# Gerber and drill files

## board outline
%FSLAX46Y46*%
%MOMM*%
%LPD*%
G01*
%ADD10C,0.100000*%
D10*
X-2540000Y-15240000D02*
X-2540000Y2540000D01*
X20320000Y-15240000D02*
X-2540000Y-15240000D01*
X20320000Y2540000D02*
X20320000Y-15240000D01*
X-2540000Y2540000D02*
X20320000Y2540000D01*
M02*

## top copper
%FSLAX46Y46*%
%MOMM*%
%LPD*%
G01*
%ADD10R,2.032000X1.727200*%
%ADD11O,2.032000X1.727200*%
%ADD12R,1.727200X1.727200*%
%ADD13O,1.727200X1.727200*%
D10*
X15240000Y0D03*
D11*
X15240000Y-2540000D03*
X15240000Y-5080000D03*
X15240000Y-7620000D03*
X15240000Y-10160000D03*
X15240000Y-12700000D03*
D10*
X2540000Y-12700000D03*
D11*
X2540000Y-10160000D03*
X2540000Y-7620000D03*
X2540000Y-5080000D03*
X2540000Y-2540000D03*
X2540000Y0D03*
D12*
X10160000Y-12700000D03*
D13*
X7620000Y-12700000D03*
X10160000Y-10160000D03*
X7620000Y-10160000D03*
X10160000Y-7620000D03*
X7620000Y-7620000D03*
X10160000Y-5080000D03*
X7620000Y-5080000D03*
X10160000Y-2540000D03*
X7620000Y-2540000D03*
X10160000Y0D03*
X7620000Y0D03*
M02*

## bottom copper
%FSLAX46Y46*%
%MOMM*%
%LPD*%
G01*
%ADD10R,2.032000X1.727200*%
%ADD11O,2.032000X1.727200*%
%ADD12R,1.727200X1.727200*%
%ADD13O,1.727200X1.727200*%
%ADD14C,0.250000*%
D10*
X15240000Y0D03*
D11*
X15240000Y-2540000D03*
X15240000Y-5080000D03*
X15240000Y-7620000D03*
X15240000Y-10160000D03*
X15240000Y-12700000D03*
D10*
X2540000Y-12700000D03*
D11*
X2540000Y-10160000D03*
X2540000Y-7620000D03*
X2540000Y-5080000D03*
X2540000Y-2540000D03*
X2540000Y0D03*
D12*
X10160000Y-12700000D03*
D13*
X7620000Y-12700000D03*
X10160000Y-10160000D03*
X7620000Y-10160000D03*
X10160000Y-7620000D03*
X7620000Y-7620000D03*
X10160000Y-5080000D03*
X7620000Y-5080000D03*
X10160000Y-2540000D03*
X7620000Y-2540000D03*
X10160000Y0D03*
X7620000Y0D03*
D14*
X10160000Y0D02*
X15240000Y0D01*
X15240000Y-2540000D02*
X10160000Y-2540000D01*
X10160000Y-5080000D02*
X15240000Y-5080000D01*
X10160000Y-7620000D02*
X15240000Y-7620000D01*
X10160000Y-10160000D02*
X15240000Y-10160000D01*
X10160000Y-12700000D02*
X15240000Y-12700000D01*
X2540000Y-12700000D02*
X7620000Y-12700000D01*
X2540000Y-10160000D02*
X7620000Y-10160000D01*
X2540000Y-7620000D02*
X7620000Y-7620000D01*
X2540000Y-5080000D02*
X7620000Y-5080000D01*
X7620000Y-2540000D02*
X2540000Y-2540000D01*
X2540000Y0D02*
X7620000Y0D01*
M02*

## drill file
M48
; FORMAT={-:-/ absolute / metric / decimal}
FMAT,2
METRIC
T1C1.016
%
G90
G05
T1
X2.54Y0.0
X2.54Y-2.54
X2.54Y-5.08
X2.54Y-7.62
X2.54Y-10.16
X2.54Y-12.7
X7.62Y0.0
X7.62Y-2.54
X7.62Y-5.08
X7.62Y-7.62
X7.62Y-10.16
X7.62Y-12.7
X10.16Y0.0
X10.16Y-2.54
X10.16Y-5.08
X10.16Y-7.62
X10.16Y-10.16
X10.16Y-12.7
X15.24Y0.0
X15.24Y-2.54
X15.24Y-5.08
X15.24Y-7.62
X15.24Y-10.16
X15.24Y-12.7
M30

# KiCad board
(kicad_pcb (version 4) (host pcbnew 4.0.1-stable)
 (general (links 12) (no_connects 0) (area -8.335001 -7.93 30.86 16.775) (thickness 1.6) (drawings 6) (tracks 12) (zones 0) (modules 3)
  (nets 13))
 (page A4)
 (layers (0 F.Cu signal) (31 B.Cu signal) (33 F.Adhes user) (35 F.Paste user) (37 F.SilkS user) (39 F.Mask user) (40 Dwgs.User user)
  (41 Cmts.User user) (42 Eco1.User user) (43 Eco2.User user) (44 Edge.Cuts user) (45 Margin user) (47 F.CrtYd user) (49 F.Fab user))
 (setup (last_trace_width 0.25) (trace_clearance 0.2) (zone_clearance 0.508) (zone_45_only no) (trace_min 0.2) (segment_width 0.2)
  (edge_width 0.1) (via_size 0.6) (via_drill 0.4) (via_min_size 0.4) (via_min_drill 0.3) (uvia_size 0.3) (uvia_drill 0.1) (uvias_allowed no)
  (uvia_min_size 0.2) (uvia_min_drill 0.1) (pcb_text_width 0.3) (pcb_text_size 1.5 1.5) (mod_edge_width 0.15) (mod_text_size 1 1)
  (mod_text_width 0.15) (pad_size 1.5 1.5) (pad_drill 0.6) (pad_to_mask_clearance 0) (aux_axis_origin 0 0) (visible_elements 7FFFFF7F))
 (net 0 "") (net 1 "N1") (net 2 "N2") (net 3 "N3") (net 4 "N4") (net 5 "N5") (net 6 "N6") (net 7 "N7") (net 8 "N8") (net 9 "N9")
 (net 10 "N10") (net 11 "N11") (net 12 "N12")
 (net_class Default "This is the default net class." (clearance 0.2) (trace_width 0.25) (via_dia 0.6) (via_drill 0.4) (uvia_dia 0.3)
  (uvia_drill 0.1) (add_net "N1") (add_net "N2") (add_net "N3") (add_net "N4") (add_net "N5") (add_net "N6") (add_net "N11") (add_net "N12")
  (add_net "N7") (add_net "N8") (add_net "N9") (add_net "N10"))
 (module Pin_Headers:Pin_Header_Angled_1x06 (layer F.Cu) (at 15.24 0)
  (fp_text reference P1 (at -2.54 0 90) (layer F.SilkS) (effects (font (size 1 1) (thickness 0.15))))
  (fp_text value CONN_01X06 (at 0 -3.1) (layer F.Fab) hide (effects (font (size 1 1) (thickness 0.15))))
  (pad 1 thru_hole rect (at 0 0) (size 2.032 1.7272) (drill 1.016) (layers *.Cu *.Mask) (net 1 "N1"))
  (pad 2 thru_hole oval (at 0 2.54) (size 2.032 1.7272) (drill 1.016) (layers *.Cu *.Mask) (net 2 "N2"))
  (pad 3 thru_hole oval (at 0 5.08) (size 2.032 1.7272) (drill 1.016) (layers *.Cu *.Mask) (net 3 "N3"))
  (pad 4 thru_hole oval (at 0 7.62) (size 2.032 1.7272) (drill 1.016) (layers *.Cu *.Mask) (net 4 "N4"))
  (pad 5 thru_hole oval (at 0 10.16) (size 2.032 1.7272) (drill 1.016) (layers *.Cu *.Mask) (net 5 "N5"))
  (pad 6 thru_hole oval (at 0 12.7) (size 2.032 1.7272) (drill 1.016) (layers *.Cu *.Mask) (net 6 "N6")))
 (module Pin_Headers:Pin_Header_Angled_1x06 (layer F.Cu) (at 2.54 12.7 180)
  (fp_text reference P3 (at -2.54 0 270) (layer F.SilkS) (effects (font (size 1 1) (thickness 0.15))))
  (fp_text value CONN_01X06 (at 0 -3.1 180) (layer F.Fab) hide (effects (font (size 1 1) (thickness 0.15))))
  (pad 1 thru_hole rect (at 0 0 180) (size 2.032 1.7272) (drill 1.016) (layers *.Cu *.Mask) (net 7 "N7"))
  (pad 2 thru_hole oval (at 0 2.54 180) (size 2.032 1.7272) (drill 1.016) (layers *.Cu *.Mask) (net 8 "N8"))
  (pad 3 thru_hole oval (at 0 5.08 180) (size 2.032 1.7272) (drill 1.016) (layers *.Cu *.Mask) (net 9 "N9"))
  (pad 4 thru_hole oval (at 0 7.62 180) (size 2.032 1.7272) (drill 1.016) (layers *.Cu *.Mask) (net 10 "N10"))
  (pad 5 thru_hole oval (at 0 10.16 180) (size 2.032 1.7272) (drill 1.016) (layers *.Cu *.Mask) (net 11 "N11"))
  (pad 6 thru_hole oval (at 0 12.7 180) (size 2.032 1.7272) (drill 1.016) (layers *.Cu *.Mask) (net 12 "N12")))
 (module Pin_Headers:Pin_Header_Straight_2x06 (layer F.Cu) (at 10.16 12.7 180)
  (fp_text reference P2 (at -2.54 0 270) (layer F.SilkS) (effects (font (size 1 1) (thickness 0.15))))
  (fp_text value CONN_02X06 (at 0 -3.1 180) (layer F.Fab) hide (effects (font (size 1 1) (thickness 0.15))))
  (pad 1 thru_hole rect (at 0 0 180) (size 1.7272 1.7272) (drill 1.016) (layers *.Cu *.Mask) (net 6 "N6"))
  (pad 2 thru_hole oval (at 2.54 0 180) (size 1.7272 1.7272) (drill 1.016) (layers *.Cu *.Mask) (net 7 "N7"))
  (pad 3 thru_hole oval (at 0 2.54 180) (size 1.7272 1.7272) (drill 1.016) (layers *.Cu *.Mask) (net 5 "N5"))
  (pad 4 thru_hole oval (at 2.54 2.54 180) (size 1.7272 1.7272) (drill 1.016) (layers *.Cu *.Mask) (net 8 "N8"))
  (pad 5 thru_hole oval (at 0 5.08 180) (size 1.7272 1.7272) (drill 1.016) (layers *.Cu *.Mask) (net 4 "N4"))
  (pad 6 thru_hole oval (at 2.54 5.08 180) (size 1.7272 1.7272) (drill 1.016) (layers *.Cu *.Mask) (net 9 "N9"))
  (pad 7 thru_hole oval (at 0 7.62 180) (size 1.7272 1.7272) (drill 1.016) (layers *.Cu *.Mask) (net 3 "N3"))
  (pad 8 thru_hole oval (at 2.54 7.62 180) (size 1.7272 1.7272) (drill 1.016) (layers *.Cu *.Mask) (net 10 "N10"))
  (pad 9 thru_hole oval (at 0 10.16 180) (size 1.7272 1.7272) (drill 1.016) (layers *.Cu *.Mask) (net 2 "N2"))
  (pad 10 thru_hole oval (at 2.54 10.16 180) (size 1.7272 1.7272) (drill 1.016) (layers *.Cu *.Mask) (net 11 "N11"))
  (pad 11 thru_hole oval (at 0 12.7 180) (size 1.7272 1.7272) (drill 1.016) (layers *.Cu *.Mask) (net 1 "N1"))
  (pad 12 thru_hole oval (at 2.54 12.7 180) (size 1.7272 1.7272) (drill 1.016) (layers *.Cu *.Mask) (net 12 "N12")))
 (gr_line (start -2.54 15.24) (end -2.54 -2.54) (angle 90) (layer Edge.Cuts) (width 0.1))
 (gr_line (start 20.32 15.24) (end -2.54 15.24) (angle 90) (layer Edge.Cuts) (width 0.1))
 (gr_line (start 20.32 -2.54) (end 20.32 15.24) (angle 90) (layer Edge.Cuts) (width 0.1))
 (gr_line (start -2.54 -2.54) (end 20.32 -2.54) (angle 90) (layer Edge.Cuts) (width 0.1))
 (segment (start 10.16 0) (end 15.24 0) (width 0.25) (layer B.Cu) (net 1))
 (segment (start 15.24 2.54) (end 10.16 2.54) (width 0.25) (layer B.Cu) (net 2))
 (segment (start 10.16 5.08) (end 15.24 5.08) (width 0.25) (layer B.Cu) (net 3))
 (segment (start 10.16 7.62) (end 15.24 7.62) (width 0.25) (layer B.Cu) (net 4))
 (segment (start 10.16 10.16) (end 15.24 10.16) (width 0.25) (layer B.Cu) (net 5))
 (segment (start 10.16 12.7) (end 15.24 12.7) (width 0.25) (layer B.Cu) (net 6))
 (segment (start 2.54 12.7) (end 7.62 12.7) (width 0.25) (layer B.Cu) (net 7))
 (segment (start 2.54 10.16) (end 7.62 10.16) (width 0.25) (layer B.Cu) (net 8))
 (segment (start 2.54 7.62) (end 7.62 7.62) (width 0.25) (layer B.Cu) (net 9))
 (segment (start 2.54 5.08) (end 7.62 5.08) (width 0.25) (layer B.Cu) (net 10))
 (segment (start 7.62 2.54) (end 2.54 2.54) (width 0.25) (layer B.Cu) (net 11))
 (segment (start 2.54 0) (end 7.62 0) (width 0.25) (layer B.Cu) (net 12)))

